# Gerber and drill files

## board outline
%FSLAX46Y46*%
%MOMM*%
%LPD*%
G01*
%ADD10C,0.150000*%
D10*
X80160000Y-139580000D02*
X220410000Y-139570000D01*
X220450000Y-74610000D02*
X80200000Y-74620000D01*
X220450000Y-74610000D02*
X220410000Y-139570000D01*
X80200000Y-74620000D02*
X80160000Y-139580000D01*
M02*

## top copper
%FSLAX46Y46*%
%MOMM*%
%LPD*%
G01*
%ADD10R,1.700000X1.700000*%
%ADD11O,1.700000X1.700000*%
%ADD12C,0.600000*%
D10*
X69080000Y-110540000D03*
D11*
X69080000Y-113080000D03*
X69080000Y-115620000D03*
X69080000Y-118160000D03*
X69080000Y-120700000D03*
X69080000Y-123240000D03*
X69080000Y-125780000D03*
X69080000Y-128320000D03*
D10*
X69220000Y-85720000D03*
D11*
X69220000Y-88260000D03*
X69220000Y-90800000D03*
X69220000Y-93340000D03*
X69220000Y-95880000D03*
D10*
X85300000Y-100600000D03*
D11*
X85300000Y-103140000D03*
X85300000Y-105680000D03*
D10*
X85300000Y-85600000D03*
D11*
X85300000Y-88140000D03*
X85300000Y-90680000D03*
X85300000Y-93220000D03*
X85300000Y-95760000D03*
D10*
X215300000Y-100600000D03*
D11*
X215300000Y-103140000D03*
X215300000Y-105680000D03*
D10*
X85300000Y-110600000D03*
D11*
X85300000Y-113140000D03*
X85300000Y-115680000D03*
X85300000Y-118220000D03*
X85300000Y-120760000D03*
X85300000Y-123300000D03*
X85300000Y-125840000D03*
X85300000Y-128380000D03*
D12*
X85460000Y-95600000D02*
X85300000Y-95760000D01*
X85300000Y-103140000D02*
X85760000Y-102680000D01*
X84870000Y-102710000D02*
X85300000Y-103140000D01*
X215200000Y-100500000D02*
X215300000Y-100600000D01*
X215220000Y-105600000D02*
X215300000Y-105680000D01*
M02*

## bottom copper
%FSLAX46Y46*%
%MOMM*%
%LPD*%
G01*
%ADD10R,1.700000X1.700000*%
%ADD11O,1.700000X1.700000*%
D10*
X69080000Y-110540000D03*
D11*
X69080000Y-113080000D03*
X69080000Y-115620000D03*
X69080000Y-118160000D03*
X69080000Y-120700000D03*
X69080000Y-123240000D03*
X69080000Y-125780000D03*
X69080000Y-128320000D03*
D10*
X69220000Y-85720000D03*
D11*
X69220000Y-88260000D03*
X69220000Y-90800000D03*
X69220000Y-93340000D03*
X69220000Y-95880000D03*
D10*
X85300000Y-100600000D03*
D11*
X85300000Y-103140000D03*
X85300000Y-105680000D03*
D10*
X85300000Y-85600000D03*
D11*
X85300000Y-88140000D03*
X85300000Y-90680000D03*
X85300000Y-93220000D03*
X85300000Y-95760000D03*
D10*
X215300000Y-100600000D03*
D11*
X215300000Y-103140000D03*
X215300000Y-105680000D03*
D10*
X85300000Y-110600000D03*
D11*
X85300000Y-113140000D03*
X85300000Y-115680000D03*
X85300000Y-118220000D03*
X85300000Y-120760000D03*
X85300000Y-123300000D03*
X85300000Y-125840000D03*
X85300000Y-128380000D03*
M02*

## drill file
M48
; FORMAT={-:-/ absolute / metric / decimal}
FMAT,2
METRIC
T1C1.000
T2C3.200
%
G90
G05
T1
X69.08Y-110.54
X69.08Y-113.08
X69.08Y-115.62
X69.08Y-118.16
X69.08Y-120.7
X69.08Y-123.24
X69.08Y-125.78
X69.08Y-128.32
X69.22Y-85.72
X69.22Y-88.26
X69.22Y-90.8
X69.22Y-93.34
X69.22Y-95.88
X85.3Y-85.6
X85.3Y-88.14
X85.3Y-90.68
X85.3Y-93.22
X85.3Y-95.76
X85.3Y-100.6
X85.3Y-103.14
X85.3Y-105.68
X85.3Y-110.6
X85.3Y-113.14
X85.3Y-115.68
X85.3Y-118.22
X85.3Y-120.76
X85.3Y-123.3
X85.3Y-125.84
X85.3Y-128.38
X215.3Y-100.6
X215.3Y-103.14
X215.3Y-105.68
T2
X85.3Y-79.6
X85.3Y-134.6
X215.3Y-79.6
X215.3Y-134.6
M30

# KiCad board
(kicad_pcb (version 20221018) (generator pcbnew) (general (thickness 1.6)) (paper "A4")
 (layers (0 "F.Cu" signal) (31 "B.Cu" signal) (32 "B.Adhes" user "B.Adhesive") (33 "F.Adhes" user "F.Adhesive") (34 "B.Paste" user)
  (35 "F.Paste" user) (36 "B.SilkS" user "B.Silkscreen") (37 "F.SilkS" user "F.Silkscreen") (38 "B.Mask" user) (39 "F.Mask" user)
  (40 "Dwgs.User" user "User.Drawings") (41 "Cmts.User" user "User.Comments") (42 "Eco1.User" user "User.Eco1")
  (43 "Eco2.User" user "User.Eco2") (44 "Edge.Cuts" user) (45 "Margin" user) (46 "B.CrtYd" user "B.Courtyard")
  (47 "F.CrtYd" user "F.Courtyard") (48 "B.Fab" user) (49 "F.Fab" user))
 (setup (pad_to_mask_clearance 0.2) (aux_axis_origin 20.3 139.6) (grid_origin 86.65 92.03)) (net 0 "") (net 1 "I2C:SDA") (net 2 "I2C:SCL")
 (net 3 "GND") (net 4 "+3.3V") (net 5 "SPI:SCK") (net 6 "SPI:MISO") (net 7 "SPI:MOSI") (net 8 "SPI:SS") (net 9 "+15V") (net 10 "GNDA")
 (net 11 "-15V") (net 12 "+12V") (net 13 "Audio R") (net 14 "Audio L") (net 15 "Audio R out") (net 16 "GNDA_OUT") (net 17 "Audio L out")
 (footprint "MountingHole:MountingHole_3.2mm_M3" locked (layer "F.Cu") (at 85.3 79.6)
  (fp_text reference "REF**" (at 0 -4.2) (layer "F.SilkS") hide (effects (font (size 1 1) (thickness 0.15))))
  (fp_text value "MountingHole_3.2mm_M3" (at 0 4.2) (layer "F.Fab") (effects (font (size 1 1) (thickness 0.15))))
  (pad "" np_thru_hole circle locked (at 0 0) (size 3.2 3.2) (drill 3.2) (layers "*.Cu" "*.Mask")))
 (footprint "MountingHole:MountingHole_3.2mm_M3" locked (layer "F.Cu") (at 215.3 79.6)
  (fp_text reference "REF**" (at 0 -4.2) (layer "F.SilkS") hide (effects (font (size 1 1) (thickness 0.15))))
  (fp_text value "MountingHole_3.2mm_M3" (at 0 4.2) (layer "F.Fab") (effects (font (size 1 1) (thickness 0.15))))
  (pad "" np_thru_hole circle locked (at 0 0) (size 3.2 3.2) (drill 3.2) (layers "F&B.Cu" "*.Mask")))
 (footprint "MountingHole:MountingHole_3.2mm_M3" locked (layer "F.Cu") (at 215.3 134.6)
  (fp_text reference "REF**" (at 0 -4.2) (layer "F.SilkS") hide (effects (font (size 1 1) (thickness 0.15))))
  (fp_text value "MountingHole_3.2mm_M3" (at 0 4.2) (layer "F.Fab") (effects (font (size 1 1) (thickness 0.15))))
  (pad "" np_thru_hole circle locked (at 0 0) (size 3.2 3.2) (drill 3.2) (layers "F&B.Cu" "*.Mask")))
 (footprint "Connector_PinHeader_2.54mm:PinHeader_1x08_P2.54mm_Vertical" (layer "F.Cu") (at 69.08 110.54)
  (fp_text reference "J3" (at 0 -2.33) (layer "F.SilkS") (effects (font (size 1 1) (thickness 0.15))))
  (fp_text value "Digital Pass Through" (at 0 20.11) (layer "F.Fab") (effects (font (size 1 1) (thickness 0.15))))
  (pad "1" thru_hole rect (at 0 0) (size 1.7 1.7) (drill 1) (layers "*.Cu" "*.Mask") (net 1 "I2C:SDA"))
  (pad "2" thru_hole oval (at 0 2.54) (size 1.7 1.7) (drill 1) (layers "*.Cu" "*.Mask") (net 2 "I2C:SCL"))
  (pad "3" thru_hole oval (at 0 5.08) (size 1.7 1.7) (drill 1) (layers "*.Cu" "*.Mask") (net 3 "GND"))
  (pad "4" thru_hole oval (at 0 7.62) (size 1.7 1.7) (drill 1) (layers "*.Cu" "*.Mask") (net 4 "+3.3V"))
  (pad "5" thru_hole oval (at 0 10.16) (size 1.7 1.7) (drill 1) (layers "*.Cu" "*.Mask") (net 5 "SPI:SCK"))
  (pad "6" thru_hole oval (at 0 12.7) (size 1.7 1.7) (drill 1) (layers "*.Cu" "*.Mask") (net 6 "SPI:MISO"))
  (pad "7" thru_hole oval (at 0 15.24) (size 1.7 1.7) (drill 1) (layers "*.Cu" "*.Mask") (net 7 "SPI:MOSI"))
  (pad "8" thru_hole oval (at 0 17.78) (size 1.7 1.7) (drill 1) (layers "*.Cu" "*.Mask") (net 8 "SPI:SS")))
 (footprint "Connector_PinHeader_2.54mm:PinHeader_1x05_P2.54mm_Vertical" (layer "F.Cu") (at 69.22 85.72)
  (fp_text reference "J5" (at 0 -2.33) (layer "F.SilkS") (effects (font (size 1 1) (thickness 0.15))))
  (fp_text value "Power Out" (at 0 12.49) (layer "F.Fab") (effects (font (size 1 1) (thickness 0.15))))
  (pad "1" thru_hole rect (at 0 0) (size 1.7 1.7) (drill 1) (layers "*.Cu" "*.Mask") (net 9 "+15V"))
  (pad "2" thru_hole oval (at 0 2.54) (size 1.7 1.7) (drill 1) (layers "*.Cu" "*.Mask") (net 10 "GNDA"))
  (pad "3" thru_hole oval (at 0 5.08) (size 1.7 1.7) (drill 1) (layers "*.Cu" "*.Mask") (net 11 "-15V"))
  (pad "4" thru_hole oval (at 0 7.62) (size 1.7 1.7) (drill 1) (layers "*.Cu" "*.Mask") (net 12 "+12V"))
  (pad "5" thru_hole oval (at 0 10.16) (size 1.7 1.7) (drill 1) (layers "*.Cu" "*.Mask") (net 3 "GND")))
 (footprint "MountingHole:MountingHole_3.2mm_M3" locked (layer "F.Cu") (at 85.3 134.6)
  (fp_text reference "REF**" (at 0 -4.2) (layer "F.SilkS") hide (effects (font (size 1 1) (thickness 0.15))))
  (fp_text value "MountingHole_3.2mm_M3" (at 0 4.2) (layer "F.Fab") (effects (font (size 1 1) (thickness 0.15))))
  (pad "" np_thru_hole circle locked (at 0 0) (size 3.2 3.2) (drill 3.2) (layers "*.Cu" "*.Mask")))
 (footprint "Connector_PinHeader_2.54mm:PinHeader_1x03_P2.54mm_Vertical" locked (layer "B.Cu") (at 85.3 100.6 180)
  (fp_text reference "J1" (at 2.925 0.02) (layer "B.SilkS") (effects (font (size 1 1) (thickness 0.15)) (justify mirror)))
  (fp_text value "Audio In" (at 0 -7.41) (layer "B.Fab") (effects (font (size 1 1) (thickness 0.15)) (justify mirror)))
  (pad "1" thru_hole rect locked (at 0 0 180) (size 1.7 1.7) (drill 1) (layers "*.Cu" "*.Mask") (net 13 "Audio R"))
  (pad "2" thru_hole oval locked (at 0 -2.54 180) (size 1.7 1.7) (drill 1) (layers "*.Cu" "*.Mask") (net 10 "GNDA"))
  (pad "3" thru_hole oval locked (at 0 -5.08 180) (size 1.7 1.7) (drill 1) (layers "*.Cu" "*.Mask") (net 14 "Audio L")))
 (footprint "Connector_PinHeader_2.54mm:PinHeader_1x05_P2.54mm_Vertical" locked (layer "B.Cu") (at 85.3 85.6 180)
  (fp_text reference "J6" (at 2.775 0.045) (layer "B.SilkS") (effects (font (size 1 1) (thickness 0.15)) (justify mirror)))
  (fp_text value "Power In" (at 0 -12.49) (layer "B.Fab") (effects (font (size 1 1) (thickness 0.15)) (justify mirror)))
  (pad "1" thru_hole rect locked (at 0 0 180) (size 1.7 1.7) (drill 1) (layers "*.Cu" "*.Mask") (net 9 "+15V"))
  (pad "2" thru_hole oval locked (at 0 -2.54 180) (size 1.7 1.7) (drill 1) (layers "*.Cu" "*.Mask") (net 10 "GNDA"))
  (pad "3" thru_hole oval locked (at 0 -5.08 180) (size 1.7 1.7) (drill 1) (layers "*.Cu" "*.Mask") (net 11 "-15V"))
  (pad "4" thru_hole oval locked (at 0 -7.62 180) (size 1.7 1.7) (drill 1) (layers "*.Cu" "*.Mask") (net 12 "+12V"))
  (pad "5" thru_hole oval locked (at 0 -10.16 180) (size 1.7 1.7) (drill 1) (layers "*.Cu" "*.Mask") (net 3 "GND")))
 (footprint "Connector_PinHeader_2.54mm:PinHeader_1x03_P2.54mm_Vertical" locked (layer "B.Cu") (at 215.3 100.6 180)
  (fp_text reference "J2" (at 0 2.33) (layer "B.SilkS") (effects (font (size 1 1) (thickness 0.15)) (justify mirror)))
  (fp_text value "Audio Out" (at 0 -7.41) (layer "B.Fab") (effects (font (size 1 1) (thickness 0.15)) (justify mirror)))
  (pad "1" thru_hole rect locked (at 0 0 180) (size 1.7 1.7) (drill 1) (layers "*.Cu" "*.Mask") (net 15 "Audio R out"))
  (pad "2" thru_hole oval locked (at 0 -2.54 180) (size 1.7 1.7) (drill 1) (layers "*.Cu" "*.Mask") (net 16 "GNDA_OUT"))
  (pad "3" thru_hole oval locked (at 0 -5.08 180) (size 1.7 1.7) (drill 1) (layers "*.Cu" "*.Mask") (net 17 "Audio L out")))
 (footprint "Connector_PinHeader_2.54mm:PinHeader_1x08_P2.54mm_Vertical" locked (layer "B.Cu") (at 85.3 110.6 180)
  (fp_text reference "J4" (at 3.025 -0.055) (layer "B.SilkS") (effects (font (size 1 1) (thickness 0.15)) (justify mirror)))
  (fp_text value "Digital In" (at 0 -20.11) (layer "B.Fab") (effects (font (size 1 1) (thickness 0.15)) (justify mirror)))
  (pad "1" thru_hole rect locked (at 0 0 180) (size 1.7 1.7) (drill 1) (layers "*.Cu" "*.Mask") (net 1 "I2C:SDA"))
  (pad "2" thru_hole oval locked (at 0 -2.54 180) (size 1.7 1.7) (drill 1) (layers "*.Cu" "*.Mask") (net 2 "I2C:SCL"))
  (pad "3" thru_hole oval locked (at 0 -5.08 180) (size 1.7 1.7) (drill 1) (layers "*.Cu" "*.Mask") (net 3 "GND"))
  (pad "4" thru_hole oval locked (at 0 -7.62 180) (size 1.7 1.7) (drill 1) (layers "*.Cu" "*.Mask") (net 4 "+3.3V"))
  (pad "5" thru_hole oval locked (at 0 -10.16 180) (size 1.7 1.7) (drill 1) (layers "*.Cu" "*.Mask") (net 5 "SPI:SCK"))
  (pad "6" thru_hole oval locked (at 0 -12.7 180) (size 1.7 1.7) (drill 1) (layers "*.Cu" "*.Mask") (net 6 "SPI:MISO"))
  (pad "7" thru_hole oval locked (at 0 -15.24 180) (size 1.7 1.7) (drill 1) (layers "*.Cu" "*.Mask") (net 7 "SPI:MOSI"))
  (pad "8" thru_hole oval locked (at 0 -17.78 180) (size 1.7 1.7) (drill 1) (layers "*.Cu" "*.Mask") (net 8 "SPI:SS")))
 (gr_line locked (start 80.16 139.58) (end 220.41 139.57) (stroke (width 0.15) (type default)) (layer "Edge.Cuts"))
 (gr_line locked (start 220.45 74.61) (end 80.2 74.62) (stroke (width 0.15) (type default)) (layer "Edge.Cuts"))
 (gr_line locked (start 220.45 74.61) (end 220.41 139.57) (stroke (width 0.15) (type default)) (layer "Edge.Cuts"))
 (gr_line locked (start 80.2 74.62) (end 80.16 139.58) (stroke (width 0.15) (type default)) (layer "Edge.Cuts"))
 (segment locked (start 85.46 95.6) (end 85.3 95.76) (width 0.6) (layer "F.Cu") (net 3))
 (segment locked (start 85.3 103.14) (end 85.76 102.68) (width 0.6) (layer "F.Cu") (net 10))
 (segment locked (start 84.87 102.71) (end 85.3 103.14) (width 0.6) (layer "F.Cu") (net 10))
 (segment locked (start 215.2 100.5) (end 215.3 100.6) (width 0.6) (layer "F.Cu") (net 15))
 (segment locked (start 215.22 105.6) (end 215.3 105.68) (width 0.6) (layer "F.Cu") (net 17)))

